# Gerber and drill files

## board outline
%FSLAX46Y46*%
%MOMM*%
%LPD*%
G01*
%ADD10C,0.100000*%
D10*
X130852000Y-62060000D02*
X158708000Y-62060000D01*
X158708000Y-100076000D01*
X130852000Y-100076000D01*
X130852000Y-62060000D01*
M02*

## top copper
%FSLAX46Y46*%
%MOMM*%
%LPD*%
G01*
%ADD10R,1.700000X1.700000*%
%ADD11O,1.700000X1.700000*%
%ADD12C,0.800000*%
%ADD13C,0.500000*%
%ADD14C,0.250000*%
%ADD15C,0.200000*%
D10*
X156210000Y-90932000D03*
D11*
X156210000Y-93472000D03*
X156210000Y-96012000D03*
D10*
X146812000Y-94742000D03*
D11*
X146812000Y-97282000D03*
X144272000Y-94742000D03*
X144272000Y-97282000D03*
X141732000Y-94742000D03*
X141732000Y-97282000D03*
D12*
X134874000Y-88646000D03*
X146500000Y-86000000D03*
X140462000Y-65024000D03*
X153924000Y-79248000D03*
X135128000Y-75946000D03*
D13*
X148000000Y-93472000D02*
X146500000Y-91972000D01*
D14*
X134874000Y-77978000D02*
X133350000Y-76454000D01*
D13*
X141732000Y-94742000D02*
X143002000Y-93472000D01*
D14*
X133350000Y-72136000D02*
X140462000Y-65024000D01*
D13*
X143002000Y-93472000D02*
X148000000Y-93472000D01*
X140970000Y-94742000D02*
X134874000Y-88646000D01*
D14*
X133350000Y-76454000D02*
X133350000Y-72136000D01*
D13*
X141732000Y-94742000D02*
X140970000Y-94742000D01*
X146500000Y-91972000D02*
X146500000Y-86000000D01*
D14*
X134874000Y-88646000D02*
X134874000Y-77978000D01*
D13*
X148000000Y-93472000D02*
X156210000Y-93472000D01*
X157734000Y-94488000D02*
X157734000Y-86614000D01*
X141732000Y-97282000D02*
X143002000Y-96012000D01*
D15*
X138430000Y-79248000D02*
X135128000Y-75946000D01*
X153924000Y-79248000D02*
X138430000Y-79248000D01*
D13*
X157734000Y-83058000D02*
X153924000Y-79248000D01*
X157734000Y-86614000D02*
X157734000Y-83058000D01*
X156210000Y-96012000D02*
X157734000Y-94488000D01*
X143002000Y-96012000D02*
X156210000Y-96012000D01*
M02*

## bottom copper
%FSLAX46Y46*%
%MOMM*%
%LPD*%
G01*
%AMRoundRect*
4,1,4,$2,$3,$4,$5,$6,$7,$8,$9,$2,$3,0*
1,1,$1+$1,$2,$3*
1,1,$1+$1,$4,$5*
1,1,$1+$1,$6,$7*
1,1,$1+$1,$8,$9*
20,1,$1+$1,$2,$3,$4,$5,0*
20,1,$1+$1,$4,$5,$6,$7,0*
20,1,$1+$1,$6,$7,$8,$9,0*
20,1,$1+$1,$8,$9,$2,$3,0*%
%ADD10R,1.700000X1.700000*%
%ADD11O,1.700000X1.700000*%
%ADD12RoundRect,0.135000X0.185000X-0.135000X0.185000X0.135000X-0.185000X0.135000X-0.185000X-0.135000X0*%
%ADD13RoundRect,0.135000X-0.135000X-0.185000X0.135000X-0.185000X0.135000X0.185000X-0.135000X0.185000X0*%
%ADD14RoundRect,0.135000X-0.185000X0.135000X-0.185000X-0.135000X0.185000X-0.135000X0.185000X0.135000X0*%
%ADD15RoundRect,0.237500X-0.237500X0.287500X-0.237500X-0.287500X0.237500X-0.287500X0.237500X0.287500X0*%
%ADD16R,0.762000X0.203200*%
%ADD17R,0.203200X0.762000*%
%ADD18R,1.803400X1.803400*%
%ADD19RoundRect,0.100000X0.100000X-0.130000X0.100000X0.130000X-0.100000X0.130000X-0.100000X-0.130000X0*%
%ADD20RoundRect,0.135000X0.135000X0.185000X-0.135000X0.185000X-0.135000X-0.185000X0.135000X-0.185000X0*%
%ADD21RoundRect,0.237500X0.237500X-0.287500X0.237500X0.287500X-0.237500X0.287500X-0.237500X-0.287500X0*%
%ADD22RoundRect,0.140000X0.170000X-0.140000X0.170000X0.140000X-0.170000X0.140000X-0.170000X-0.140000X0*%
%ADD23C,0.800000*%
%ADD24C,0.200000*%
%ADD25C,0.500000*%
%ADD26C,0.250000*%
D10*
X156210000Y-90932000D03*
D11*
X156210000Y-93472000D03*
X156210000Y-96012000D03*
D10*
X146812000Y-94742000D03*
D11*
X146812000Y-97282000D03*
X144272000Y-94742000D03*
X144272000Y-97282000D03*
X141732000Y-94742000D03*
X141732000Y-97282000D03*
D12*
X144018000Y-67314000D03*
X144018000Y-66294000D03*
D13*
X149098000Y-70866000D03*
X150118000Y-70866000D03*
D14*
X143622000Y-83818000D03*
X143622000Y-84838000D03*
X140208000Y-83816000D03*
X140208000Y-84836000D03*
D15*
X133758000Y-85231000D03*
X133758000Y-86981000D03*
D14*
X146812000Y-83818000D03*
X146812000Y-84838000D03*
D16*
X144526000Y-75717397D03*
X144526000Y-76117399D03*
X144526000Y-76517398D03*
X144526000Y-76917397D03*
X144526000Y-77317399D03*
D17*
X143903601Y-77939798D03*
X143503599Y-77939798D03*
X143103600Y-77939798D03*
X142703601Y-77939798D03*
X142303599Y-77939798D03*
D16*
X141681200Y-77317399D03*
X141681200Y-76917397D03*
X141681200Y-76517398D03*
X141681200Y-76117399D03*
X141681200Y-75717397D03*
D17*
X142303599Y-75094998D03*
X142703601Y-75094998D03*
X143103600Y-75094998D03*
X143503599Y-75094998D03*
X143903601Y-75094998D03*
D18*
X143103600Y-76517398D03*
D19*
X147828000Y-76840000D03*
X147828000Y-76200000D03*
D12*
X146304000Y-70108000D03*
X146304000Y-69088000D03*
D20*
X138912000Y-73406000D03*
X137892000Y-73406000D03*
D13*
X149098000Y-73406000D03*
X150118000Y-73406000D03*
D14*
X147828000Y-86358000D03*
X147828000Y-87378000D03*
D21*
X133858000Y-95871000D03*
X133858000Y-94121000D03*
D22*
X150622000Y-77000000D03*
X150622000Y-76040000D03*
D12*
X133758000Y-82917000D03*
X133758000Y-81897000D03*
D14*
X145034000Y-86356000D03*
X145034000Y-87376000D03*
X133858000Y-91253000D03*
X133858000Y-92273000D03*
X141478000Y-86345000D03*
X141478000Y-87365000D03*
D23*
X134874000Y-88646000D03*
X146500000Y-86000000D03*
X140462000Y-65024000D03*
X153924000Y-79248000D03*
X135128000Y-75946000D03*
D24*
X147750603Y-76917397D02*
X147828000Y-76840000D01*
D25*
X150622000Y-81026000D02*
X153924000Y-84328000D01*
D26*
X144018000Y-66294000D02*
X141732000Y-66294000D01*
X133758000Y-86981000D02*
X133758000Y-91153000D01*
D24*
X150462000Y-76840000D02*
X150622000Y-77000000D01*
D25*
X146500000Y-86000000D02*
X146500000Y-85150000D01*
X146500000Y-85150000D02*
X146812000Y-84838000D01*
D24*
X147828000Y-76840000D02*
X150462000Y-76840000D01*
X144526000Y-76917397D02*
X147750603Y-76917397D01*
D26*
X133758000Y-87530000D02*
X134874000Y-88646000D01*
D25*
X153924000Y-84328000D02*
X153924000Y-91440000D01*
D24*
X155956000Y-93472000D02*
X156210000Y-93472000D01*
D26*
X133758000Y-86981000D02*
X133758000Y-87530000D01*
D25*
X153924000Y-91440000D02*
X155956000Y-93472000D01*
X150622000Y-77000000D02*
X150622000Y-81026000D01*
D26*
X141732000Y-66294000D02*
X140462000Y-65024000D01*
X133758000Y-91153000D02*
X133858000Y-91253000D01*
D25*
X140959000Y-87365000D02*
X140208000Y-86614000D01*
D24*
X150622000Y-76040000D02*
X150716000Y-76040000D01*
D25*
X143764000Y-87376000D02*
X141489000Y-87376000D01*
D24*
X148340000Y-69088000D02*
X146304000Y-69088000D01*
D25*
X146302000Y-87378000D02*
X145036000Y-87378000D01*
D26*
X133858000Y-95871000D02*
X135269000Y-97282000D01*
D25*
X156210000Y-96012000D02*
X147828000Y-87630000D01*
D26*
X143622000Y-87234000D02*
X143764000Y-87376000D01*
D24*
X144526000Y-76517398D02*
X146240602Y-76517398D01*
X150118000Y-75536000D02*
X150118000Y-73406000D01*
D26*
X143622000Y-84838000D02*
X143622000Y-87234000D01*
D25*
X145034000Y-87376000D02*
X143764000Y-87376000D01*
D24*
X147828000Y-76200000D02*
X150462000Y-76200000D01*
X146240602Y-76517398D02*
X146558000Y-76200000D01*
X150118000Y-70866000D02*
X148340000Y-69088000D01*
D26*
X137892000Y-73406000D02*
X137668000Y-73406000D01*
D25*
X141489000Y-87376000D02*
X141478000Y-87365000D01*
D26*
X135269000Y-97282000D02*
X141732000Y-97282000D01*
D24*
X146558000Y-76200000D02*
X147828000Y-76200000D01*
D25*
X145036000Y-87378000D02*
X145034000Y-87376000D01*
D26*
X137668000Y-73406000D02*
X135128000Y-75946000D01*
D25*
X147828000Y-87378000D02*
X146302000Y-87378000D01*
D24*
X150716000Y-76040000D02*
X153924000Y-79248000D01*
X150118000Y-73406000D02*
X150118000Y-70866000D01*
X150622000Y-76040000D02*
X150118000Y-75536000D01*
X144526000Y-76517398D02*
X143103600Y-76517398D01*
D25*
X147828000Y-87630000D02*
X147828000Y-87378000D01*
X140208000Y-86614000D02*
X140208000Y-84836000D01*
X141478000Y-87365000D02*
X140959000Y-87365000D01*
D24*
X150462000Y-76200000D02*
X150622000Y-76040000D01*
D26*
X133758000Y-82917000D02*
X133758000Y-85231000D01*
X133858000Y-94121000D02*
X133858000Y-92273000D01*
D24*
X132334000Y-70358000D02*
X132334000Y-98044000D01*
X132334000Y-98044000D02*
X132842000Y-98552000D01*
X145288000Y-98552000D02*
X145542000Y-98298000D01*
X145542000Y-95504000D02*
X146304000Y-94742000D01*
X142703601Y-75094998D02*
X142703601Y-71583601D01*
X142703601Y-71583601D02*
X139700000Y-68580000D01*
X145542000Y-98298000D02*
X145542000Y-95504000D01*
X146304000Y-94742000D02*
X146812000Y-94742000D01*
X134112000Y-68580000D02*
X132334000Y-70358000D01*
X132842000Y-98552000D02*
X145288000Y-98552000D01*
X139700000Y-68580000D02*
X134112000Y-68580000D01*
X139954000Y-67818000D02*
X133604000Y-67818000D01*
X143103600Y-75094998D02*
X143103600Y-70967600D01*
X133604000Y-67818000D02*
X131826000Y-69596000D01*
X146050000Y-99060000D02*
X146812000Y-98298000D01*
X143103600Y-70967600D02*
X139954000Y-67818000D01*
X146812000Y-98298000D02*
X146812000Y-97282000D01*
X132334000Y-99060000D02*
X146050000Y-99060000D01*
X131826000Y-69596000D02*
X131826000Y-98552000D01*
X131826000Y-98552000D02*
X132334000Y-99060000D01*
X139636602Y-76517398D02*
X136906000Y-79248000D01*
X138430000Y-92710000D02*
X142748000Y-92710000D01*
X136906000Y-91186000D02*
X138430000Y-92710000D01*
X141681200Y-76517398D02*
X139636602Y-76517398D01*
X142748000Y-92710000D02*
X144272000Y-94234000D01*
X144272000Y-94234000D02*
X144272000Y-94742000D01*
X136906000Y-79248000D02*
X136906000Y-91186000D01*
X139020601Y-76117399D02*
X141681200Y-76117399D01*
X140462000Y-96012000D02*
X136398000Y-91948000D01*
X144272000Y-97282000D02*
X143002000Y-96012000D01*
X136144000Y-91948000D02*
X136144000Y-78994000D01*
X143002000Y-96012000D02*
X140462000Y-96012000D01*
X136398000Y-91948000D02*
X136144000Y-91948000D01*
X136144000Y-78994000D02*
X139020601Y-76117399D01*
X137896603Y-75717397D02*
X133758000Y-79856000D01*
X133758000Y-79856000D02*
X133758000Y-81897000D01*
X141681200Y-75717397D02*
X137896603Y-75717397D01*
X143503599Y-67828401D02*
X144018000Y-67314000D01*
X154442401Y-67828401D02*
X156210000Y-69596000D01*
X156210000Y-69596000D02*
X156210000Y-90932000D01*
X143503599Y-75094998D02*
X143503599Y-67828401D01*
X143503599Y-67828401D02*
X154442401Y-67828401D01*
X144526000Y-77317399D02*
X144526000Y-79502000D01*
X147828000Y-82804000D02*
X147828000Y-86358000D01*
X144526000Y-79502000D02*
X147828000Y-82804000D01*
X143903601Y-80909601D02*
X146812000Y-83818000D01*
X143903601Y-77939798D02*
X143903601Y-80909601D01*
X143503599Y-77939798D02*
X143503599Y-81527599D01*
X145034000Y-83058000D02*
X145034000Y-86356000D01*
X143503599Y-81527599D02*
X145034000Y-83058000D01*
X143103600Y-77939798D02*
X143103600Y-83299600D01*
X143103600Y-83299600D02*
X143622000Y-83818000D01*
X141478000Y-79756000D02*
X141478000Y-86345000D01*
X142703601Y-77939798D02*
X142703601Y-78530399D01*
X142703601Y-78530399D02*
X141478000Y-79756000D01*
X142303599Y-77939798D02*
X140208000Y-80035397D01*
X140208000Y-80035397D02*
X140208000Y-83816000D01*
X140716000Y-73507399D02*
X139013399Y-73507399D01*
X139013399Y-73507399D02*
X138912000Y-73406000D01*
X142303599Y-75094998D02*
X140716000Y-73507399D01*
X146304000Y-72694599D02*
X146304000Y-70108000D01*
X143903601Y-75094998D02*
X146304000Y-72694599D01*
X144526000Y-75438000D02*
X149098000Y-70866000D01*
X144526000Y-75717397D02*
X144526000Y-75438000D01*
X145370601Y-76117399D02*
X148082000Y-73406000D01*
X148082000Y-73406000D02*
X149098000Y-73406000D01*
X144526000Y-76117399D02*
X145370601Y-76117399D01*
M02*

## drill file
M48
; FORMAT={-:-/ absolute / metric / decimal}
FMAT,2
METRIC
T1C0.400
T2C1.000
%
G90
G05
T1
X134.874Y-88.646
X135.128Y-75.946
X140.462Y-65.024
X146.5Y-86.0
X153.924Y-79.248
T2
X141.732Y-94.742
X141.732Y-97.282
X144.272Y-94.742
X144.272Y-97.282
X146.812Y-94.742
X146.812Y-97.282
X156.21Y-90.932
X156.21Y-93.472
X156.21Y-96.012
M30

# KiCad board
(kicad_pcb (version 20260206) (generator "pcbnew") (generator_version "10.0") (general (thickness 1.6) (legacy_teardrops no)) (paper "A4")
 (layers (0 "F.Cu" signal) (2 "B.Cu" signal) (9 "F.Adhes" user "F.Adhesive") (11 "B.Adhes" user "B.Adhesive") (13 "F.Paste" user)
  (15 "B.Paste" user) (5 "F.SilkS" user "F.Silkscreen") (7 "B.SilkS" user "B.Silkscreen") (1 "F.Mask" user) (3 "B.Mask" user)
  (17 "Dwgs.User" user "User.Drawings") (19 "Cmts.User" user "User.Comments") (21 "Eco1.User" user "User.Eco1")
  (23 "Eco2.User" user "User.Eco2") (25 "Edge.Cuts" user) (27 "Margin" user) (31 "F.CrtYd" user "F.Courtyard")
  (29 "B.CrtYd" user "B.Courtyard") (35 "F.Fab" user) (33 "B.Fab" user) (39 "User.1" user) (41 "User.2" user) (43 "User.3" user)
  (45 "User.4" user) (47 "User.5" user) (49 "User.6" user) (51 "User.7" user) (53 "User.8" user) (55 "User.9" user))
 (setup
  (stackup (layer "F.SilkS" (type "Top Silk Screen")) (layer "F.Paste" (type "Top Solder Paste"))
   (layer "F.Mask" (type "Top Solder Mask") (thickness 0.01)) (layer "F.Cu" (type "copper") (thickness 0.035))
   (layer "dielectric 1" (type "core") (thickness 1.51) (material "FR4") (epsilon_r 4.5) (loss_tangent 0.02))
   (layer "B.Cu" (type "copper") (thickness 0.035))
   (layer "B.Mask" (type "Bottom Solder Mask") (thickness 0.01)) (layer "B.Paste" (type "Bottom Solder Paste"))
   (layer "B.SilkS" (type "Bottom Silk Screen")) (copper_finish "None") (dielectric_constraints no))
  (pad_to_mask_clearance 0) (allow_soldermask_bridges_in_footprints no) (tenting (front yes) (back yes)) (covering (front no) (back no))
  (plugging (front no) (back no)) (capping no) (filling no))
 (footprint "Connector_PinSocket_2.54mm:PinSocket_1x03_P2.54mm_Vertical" (layer "F.Cu") (at 156.21 90.932)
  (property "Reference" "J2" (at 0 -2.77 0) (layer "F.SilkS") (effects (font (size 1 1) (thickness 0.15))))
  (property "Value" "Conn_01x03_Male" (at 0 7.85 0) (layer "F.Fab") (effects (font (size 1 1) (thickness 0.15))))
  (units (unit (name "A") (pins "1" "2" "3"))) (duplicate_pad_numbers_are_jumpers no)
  (pad "1" thru_hole rect (at 0 0) (size 1.7 1.7) (drill 1) (layers "*.Cu" "*.Mask") (remove_unused_layers no) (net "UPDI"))
  (pad "2" thru_hole oval (at 0 2.54) (size 1.7 1.7) (drill 1) (layers "*.Cu" "*.Mask") (remove_unused_layers no) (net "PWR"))
  (pad "3" thru_hole oval (at 0 5.08) (size 1.7 1.7) (drill 1) (layers "*.Cu" "*.Mask") (remove_unused_layers no) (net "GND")))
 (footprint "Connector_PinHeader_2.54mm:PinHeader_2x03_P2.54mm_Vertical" (layer "F.Cu") (at 146.812 94.742 -90)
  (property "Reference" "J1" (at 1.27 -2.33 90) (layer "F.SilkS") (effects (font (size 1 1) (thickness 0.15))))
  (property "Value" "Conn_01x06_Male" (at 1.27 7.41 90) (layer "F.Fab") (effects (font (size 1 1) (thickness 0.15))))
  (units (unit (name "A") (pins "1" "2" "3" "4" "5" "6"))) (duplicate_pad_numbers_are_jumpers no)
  (pad "1" thru_hole rect (at 0 0 270) (size 1.7 1.7) (drill 1) (layers "*.Cu" "*.Mask") (remove_unused_layers no) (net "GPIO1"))
  (pad "2" thru_hole oval (at 2.54 0 270) (size 1.7 1.7) (drill 1) (layers "*.Cu" "*.Mask") (remove_unused_layers no) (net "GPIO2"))
  (pad "3" thru_hole oval (at 0 2.54 270) (size 1.7 1.7) (drill 1) (layers "*.Cu" "*.Mask") (remove_unused_layers no) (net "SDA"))
  (pad "4" thru_hole oval (at 2.54 2.54 270) (size 1.7 1.7) (drill 1) (layers "*.Cu" "*.Mask") (remove_unused_layers no) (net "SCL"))
  (pad "5" thru_hole oval (at 0 5.08 270) (size 1.7 1.7) (drill 1) (layers "*.Cu" "*.Mask") (remove_unused_layers no) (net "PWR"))
  (pad "6" thru_hole oval (at 2.54 5.08 270) (size 1.7 1.7) (drill 1) (layers "*.Cu" "*.Mask") (remove_unused_layers no) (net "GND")))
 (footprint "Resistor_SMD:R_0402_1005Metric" (layer "B.Cu") (at 144.018 66.804 90)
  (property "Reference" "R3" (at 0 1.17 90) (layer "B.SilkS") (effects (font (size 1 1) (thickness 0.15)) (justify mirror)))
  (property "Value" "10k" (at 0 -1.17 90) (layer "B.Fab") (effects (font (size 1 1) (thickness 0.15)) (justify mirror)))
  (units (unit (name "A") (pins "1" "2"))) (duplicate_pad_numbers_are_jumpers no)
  (pad "1" smd roundrect (at -0.51 0 90) (size 0.54 0.64) (layers "B.Cu" "B.Mask" "B.Paste") (roundrect_rratio 0.25) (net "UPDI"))
  (pad "2" smd roundrect (at 0.51 0 90) (size 0.54 0.64) (layers "B.Cu" "B.Mask" "B.Paste") (roundrect_rratio 0.25) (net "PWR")))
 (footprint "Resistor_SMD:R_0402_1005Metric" (layer "B.Cu") (at 149.608 70.866)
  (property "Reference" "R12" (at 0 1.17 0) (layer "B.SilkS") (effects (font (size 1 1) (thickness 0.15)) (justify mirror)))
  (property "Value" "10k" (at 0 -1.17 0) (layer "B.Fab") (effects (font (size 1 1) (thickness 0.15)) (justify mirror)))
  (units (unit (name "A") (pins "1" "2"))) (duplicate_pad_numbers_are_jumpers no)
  (pad "1" smd roundrect (at -0.51 0) (size 0.54 0.64) (layers "B.Cu" "B.Mask" "B.Paste") (roundrect_rratio 0.25) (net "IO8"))
  (pad "2" smd roundrect (at 0.51 0) (size 0.54 0.64) (layers "B.Cu" "B.Mask" "B.Paste") (roundrect_rratio 0.25) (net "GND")))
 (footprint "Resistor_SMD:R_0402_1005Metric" (layer "B.Cu") (at 143.622 84.328 -90)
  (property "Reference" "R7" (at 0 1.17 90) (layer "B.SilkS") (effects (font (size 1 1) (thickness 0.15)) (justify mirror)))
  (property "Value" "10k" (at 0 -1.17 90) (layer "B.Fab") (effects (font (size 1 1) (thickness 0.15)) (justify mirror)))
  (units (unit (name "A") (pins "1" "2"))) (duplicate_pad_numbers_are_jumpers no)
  (pad "1" smd roundrect (at -0.51 0 270) (size 0.54 0.64) (layers "B.Cu" "B.Mask" "B.Paste") (roundrect_rratio 0.25) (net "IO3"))
  (pad "2" smd roundrect (at 0.51 0 270) (size 0.54 0.64) (layers "B.Cu" "B.Mask" "B.Paste") (roundrect_rratio 0.25) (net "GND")))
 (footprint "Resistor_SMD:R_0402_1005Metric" (layer "B.Cu") (at 140.208 84.326 -90)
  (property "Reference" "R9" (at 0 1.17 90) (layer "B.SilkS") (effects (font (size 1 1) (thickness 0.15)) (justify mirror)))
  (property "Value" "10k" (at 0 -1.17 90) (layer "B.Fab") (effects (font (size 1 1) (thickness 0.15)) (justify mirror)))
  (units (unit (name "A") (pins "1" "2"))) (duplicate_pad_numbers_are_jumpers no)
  (pad "1" smd roundrect (at -0.51 0 270) (size 0.54 0.64) (layers "B.Cu" "B.Mask" "B.Paste") (roundrect_rratio 0.25) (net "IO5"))
  (pad "2" smd roundrect (at 0.51 0 270) (size 0.54 0.64) (layers "B.Cu" "B.Mask" "B.Paste") (roundrect_rratio 0.25) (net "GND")))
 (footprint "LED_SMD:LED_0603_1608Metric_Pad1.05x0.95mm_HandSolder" (layer "B.Cu") (at 133.758 86.106 -90)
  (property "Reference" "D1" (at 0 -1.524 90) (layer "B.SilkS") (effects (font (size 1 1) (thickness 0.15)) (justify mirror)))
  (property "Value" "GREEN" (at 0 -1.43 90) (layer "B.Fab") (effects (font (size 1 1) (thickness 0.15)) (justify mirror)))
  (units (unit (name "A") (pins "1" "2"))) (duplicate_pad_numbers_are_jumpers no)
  (pad "1" smd roundrect (at -0.875 0 270) (size 1.05 0.95) (layers "B.Cu" "B.Mask" "B.Paste") (roundrect_rratio 0.25) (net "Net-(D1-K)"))
  (pad "2" smd roundrect (at 0.875 0 270) (size 1.05 0.95) (layers "B.Cu" "B.Mask" "B.Paste") (roundrect_rratio 0.25) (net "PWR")))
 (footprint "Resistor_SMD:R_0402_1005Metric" (layer "B.Cu") (at 146.812 84.328 -90)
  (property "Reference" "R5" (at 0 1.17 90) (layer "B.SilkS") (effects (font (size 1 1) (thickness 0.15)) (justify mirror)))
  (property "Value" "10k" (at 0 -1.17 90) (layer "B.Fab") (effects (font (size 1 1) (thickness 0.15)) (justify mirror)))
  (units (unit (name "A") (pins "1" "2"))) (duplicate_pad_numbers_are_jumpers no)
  (pad "1" smd roundrect (at -0.51 0 270) (size 0.54 0.64) (layers "B.Cu" "B.Mask" "B.Paste") (roundrect_rratio 0.25) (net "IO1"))
  (pad "2" smd roundrect (at 0.51 0 270) (size 0.54 0.64) (layers "B.Cu" "B.Mask" "B.Paste") (roundrect_rratio 0.25) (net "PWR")))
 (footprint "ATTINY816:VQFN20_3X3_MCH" (layer "B.Cu") (at 143.1036 76.517398 180)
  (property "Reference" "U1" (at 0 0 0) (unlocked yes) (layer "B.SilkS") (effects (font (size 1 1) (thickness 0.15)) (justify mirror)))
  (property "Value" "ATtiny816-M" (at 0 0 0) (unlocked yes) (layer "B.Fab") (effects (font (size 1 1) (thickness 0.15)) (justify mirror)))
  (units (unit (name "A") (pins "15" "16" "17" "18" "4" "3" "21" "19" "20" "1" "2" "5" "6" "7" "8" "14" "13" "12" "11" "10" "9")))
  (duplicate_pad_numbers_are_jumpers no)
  (pad "1" smd rect (at -1.4224 0.800001 90) (size 0.2032 0.762) (layers "B.Cu" "B.Mask" "B.Paste") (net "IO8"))
  (pad "2" smd rect (at -1.4224 0.399999 90) (size 0.2032 0.762) (layers "B.Cu" "B.Mask" "B.Paste") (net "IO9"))
  (pad "3" smd rect (at -1.4224 0 90) (size 0.2032 0.762) (layers "B.Cu" "B.Mask" "B.Paste") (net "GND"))
  (pad "4" smd rect (at -1.4224 -0.399999 90) (size 0.2032 0.762) (layers "B.Cu" "B.Mask" "B.Paste") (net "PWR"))
  (pad "5" smd rect (at -1.4224 -0.800001 90) (size 0.2032 0.762) (layers "B.Cu" "B.Mask" "B.Paste") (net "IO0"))
  (pad "6" smd rect (at -0.800001 -1.4224 180) (size 0.2032 0.762) (layers "B.Cu" "B.Mask" "B.Paste") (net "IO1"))
  (pad "7" smd rect (at -0.399999 -1.4224 180) (size 0.2032 0.762) (layers "B.Cu" "B.Mask" "B.Paste") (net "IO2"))
  (pad "8" smd rect (at 0 -1.4224 180) (size 0.2032 0.762) (layers "B.Cu" "B.Mask" "B.Paste") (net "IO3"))
  (pad "9" smd rect (at 0.399999 -1.4224 180) (size 0.2032 0.762) (layers "B.Cu" "B.Mask" "B.Paste") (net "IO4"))
  (pad "10" smd rect (at 0.800001 -1.4224 180) (size 0.2032 0.762) (layers "B.Cu" "B.Mask" "B.Paste") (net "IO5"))
  (pad "11" smd rect (at 1.4224 -0.800001 90) (size 0.2032 0.762) (layers "B.Cu" "B.Mask" "B.Paste") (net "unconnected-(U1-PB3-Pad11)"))
  (pad "12" smd rect (at 1.4224 -0.399999 90) (size 0.2032 0.762) (layers "B.Cu" "B.Mask" "B.Paste") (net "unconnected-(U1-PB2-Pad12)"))
  (pad "13" smd rect (at 1.4224 0 90) (size 0.2032 0.762) (layers "B.Cu" "B.Mask" "B.Paste") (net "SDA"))
  (pad "14" smd rect (at 1.4224 0.399999 90) (size 0.2032 0.762) (layers "B.Cu" "B.Mask" "B.Paste") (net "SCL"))
  (pad "15" smd rect (at 1.4224 0.800001 90) (size 0.2032 0.762) (layers "B.Cu" "B.Mask" "B.Paste") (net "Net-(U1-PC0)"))
  (pad "16" smd rect (at 0.800001 1.4224 180) (size 0.2032 0.762) (layers "B.Cu" "B.Mask" "B.Paste") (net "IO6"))
  (pad "17" smd rect (at 0.399999 1.4224 180) (size 0.2032 0.762) (layers "B.Cu" "B.Mask" "B.Paste") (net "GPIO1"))
  (pad "18" smd rect (at 0 1.4224 180) (size 0.2032 0.762) (layers "B.Cu" "B.Mask" "B.Paste") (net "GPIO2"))
  (pad "19" smd rect (at -0.399999 1.4224 180) (size 0.2032 0.762) (layers "B.Cu" "B.Mask" "B.Paste") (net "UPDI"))
  (pad "20" smd rect (at -0.800001 1.4224 180) (size 0.2032 0.762) (layers "B.Cu" "B.Mask" "B.Paste") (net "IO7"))
  (pad "21" smd rect (at 0 0 180) (size 1.8034 1.8034) (layers "B.Cu" "B.Mask" "B.Paste") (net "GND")))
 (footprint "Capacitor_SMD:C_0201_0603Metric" (layer "B.Cu") (at 147.828 76.52 90)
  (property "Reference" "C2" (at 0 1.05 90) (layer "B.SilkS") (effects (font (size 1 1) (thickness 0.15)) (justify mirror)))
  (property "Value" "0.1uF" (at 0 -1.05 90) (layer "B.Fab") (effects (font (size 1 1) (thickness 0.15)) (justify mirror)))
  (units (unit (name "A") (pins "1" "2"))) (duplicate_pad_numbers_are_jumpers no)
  (pad "" smd roundrect (at -0.345 0 90) (size 0.318 0.36) (layers "B.Paste") (roundrect_rratio 0.25))
  (pad "" smd roundrect (at 0.345 0 90) (size 0.318 0.36) (layers "B.Paste") (roundrect_rratio 0.25))
  (pad "1" smd roundrect (at -0.32 0 90) (size 0.46 0.4) (layers "B.Cu" "B.Mask") (roundrect_rratio 0.25) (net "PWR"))
  (pad "2" smd roundrect (at 0.32 0 90) (size 0.46 0.4) (layers "B.Cu" "B.Mask") (roundrect_rratio 0.25) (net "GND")))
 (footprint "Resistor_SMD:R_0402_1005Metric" (layer "B.Cu") (at 146.304 69.598 90)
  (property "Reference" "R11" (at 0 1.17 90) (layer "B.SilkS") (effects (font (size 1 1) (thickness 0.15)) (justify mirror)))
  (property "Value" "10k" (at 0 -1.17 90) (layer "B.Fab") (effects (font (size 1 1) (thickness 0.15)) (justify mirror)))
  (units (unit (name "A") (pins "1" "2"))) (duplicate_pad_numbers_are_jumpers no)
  (pad "1" smd roundrect (at -0.51 0 90) (size 0.54 0.64) (layers "B.Cu" "B.Mask" "B.Paste") (roundrect_rratio 0.25) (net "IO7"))
  (pad "2" smd roundrect (at 0.51 0 90) (size 0.54 0.64) (layers "B.Cu" "B.Mask" "B.Paste") (roundrect_rratio 0.25) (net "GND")))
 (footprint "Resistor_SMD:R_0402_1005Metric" (layer "B.Cu") (at 138.402 73.406 180)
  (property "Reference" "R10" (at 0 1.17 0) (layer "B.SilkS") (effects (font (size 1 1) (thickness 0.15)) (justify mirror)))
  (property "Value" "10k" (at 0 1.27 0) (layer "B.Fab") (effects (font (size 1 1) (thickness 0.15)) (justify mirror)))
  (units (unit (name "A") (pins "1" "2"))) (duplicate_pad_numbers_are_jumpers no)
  (pad "1" smd roundrect (at -0.51 0 180) (size 0.54 0.64) (layers "B.Cu" "B.Mask" "B.Paste") (roundrect_rratio 0.25) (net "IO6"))
  (pad "2" smd roundrect (at 0.51 0 180) (size 0.54 0.64) (layers "B.Cu" "B.Mask" "B.Paste") (roundrect_rratio 0.25) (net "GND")))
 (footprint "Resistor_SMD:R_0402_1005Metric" (layer "B.Cu") (at 149.608 73.406)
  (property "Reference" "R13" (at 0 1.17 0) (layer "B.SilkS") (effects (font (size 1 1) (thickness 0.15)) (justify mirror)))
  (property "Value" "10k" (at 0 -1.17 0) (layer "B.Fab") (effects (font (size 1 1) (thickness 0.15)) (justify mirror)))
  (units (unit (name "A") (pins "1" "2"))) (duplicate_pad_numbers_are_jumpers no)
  (pad "1" smd roundrect (at -0.51 0) (size 0.54 0.64) (layers "B.Cu" "B.Mask" "B.Paste") (roundrect_rratio 0.25) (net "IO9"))
  (pad "2" smd roundrect (at 0.51 0) (size 0.54 0.64) (layers "B.Cu" "B.Mask" "B.Paste") (roundrect_rratio 0.25) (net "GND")))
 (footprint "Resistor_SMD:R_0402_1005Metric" (layer "B.Cu") (at 147.828 86.868 -90)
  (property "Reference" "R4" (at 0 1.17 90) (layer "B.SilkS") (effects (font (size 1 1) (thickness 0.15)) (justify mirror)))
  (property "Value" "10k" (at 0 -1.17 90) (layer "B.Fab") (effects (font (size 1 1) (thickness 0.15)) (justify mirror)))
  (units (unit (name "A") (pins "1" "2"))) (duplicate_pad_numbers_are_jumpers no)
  (pad "1" smd roundrect (at -0.51 0 270) (size 0.54 0.64) (layers "B.Cu" "B.Mask" "B.Paste") (roundrect_rratio 0.25) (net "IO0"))
  (pad "2" smd roundrect (at 0.51 0 270) (size 0.54 0.64) (layers "B.Cu" "B.Mask" "B.Paste") (roundrect_rratio 0.25) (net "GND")))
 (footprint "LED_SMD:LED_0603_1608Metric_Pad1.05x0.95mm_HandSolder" (layer "B.Cu") (at 133.858 94.996 90)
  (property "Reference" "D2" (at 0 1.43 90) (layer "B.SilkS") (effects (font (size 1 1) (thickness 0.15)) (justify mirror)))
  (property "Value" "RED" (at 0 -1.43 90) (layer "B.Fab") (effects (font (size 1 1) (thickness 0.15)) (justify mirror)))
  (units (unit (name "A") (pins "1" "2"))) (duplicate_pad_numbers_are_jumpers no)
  (pad "1" smd roundrect (at -0.875 0 90) (size 1.05 0.95) (layers "B.Cu" "B.Mask" "B.Paste") (roundrect_rratio 0.25) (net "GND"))
  (pad "2" smd roundrect (at 0.875 0 90) (size 1.05 0.95) (layers "B.Cu" "B.Mask" "B.Paste") (roundrect_rratio 0.25) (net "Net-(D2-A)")))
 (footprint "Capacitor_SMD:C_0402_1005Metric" (layer "B.Cu") (at 150.622 76.52 90)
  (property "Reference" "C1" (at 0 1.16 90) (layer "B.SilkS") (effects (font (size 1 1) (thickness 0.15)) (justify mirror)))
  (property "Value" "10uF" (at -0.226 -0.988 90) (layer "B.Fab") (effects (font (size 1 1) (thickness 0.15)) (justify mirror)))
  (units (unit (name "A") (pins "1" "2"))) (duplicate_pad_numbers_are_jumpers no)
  (pad "1" smd roundrect (at -0.48 0 90) (size 0.56 0.62) (layers "B.Cu" "B.Mask" "B.Paste") (roundrect_rratio 0.25) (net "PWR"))
  (pad "2" smd roundrect (at 0.48 0 90) (size 0.56 0.62) (layers "B.Cu" "B.Mask" "B.Paste") (roundrect_rratio 0.25) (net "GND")))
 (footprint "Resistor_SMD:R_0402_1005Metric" (layer "B.Cu") (at 133.758 82.407 90)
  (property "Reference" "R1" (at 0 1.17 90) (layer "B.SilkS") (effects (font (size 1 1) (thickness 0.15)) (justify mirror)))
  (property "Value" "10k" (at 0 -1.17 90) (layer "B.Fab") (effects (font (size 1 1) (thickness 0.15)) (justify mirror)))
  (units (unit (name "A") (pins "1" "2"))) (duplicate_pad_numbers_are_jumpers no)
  (pad "1" smd roundrect (at -0.51 0 90) (size 0.54 0.64) (layers "B.Cu" "B.Mask" "B.Paste") (roundrect_rratio 0.25) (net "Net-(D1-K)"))
  (pad "2" smd roundrect (at 0.51 0 90) (size 0.54 0.64) (layers "B.Cu" "B.Mask" "B.Paste") (roundrect_rratio 0.25) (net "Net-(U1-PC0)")))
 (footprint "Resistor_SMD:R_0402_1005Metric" (layer "B.Cu") (at 145.034 86.866 -90)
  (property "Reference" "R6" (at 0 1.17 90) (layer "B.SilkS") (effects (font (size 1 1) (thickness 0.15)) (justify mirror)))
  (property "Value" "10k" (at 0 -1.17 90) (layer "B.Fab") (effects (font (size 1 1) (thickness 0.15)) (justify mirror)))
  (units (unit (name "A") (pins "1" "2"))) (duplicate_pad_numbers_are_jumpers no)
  (pad "1" smd roundrect (at -0.51 0 270) (size 0.54 0.64) (layers "B.Cu" "B.Mask" "B.Paste") (roundrect_rratio 0.25) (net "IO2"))
  (pad "2" smd roundrect (at 0.51 0 270) (size 0.54 0.64) (layers "B.Cu" "B.Mask" "B.Paste") (roundrect_rratio 0.25) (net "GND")))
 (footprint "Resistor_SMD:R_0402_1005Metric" (layer "B.Cu") (at 133.858 91.763 -90)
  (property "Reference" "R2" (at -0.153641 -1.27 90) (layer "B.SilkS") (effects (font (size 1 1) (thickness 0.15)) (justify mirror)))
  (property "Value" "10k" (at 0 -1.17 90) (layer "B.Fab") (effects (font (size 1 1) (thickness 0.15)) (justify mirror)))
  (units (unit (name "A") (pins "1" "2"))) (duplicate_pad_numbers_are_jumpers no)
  (pad "1" smd roundrect (at -0.51 0 270) (size 0.54 0.64) (layers "B.Cu" "B.Mask" "B.Paste") (roundrect_rratio 0.25) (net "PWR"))
  (pad "2" smd roundrect (at 0.51 0 270) (size 0.54 0.64) (layers "B.Cu" "B.Mask" "B.Paste") (roundrect_rratio 0.25) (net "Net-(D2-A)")))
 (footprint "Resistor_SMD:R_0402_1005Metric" (layer "B.Cu") (at 141.478 86.855 -90)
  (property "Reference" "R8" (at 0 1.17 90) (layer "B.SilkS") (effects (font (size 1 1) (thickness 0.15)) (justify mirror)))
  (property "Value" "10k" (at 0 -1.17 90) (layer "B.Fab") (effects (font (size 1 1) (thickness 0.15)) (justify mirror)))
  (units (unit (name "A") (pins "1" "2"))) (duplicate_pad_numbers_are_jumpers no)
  (pad "1" smd roundrect (at -0.51 0 270) (size 0.54 0.64) (layers "B.Cu" "B.Mask" "B.Paste") (roundrect_rratio 0.25) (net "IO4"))
  (pad "2" smd roundrect (at 0.51 0 270) (size 0.54 0.64) (layers "B.Cu" "B.Mask" "B.Paste") (roundrect_rratio 0.25) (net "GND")))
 (gr_rect (start 130.852 62.06) (end 158.708 100.076) (stroke (width 0.1) (type solid)) (fill no) (layer "Edge.Cuts"))
 (via (at 134.874 88.646) (size 0.8) (drill 0.4) (layers "F.Cu" "B.Cu") (free yes) (capping no) (covering (front no) (back no))
  (plugging (front no) (back no)) (filling no) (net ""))
 (segment (start 148 93.472) (end 146.5 91.972) (width 0.5) (layer "F.Cu") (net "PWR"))
 (segment (start 134.874 77.978) (end 133.35 76.454) (width 0.25) (layer "F.Cu") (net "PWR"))
 (segment (start 141.732 94.742) (end 143.002 93.472) (width 0.5) (layer "F.Cu") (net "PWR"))
 (segment (start 133.35 72.136) (end 140.462 65.024) (width 0.25) (layer "F.Cu") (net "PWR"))
 (segment (start 143.002 93.472) (end 148 93.472) (width 0.5) (layer "F.Cu") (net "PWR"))
 (segment (start 140.97 94.742) (end 134.874 88.646) (width 0.5) (layer "F.Cu") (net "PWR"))
 (segment (start 133.35 76.454) (end 133.35 72.136) (width 0.25) (layer "F.Cu") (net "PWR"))
 (segment (start 141.732 94.742) (end 140.97 94.742) (width 0.5) (layer "F.Cu") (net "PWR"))
 (segment (start 146.5 91.972) (end 146.5 86) (width 0.5) (layer "F.Cu") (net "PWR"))
 (segment (start 134.874 88.646) (end 134.874 77.978) (width 0.25) (layer "F.Cu") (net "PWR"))
 (segment (start 148 93.472) (end 156.21 93.472) (width 0.5) (layer "F.Cu") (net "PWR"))
 (via (at 146.5 86) (size 0.8) (drill 0.4) (layers "F.Cu" "B.Cu") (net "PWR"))
 (via (at 140.462 65.024) (size 0.8) (drill 0.4) (layers "F.Cu" "B.Cu") (capping no) (covering (front no) (back no))
  (plugging (front no) (back no)) (filling no) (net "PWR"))
 (segment (start 147.750603 76.917397) (end 147.828 76.84) (width 0.2) (layer "B.Cu") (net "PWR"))
 (segment (start 150.622 81.026) (end 153.924 84.328) (width 0.5) (layer "B.Cu") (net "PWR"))
 (segment (start 144.018 66.294) (end 141.732 66.294) (width 0.25) (layer "B.Cu") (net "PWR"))
 (segment (start 133.758 86.981) (end 133.758 91.153) (width 0.25) (layer "B.Cu") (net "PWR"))
 (segment (start 150.462 76.84) (end 150.622 77) (width 0.2) (layer "B.Cu") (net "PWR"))
 (segment (start 146.5 86) (end 146.5 85.15) (width 0.5) (layer "B.Cu") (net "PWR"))
 (segment (start 146.5 85.15) (end 146.812 84.838) (width 0.5) (layer "B.Cu") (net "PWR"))
 (segment (start 147.828 76.84) (end 150.462 76.84) (width 0.2) (layer "B.Cu") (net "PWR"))
 (segment (start 144.526 76.917397) (end 147.750603 76.917397) (width 0.2) (layer "B.Cu") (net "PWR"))
 (segment (start 133.758 87.53) (end 134.874 88.646) (width 0.25) (layer "B.Cu") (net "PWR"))
 (segment (start 153.924 84.328) (end 153.924 91.44) (width 0.5) (layer "B.Cu") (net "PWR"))
 (segment (start 155.956 93.472) (end 156.21 93.472) (width 0.2) (layer "B.Cu") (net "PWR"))
 (segment (start 133.758 86.981) (end 133.758 87.53) (width 0.25) (layer "B.Cu") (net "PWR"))
 (segment (start 153.924 91.44) (end 155.956 93.472) (width 0.5) (layer "B.Cu") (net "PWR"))
 (segment (start 150.622 77) (end 150.622 81.026) (width 0.5) (layer "B.Cu") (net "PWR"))
 (segment (start 141.732 66.294) (end 140.462 65.024) (width 0.25) (layer "B.Cu") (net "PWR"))
 (segment (start 133.758 91.153) (end 133.858 91.253) (width 0.25) (layer "B.Cu") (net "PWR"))
 (segment (start 157.734 94.488) (end 157.734 86.614) (width 0.5) (layer "F.Cu") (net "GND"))
 (segment (start 141.732 97.282) (end 143.002 96.012) (width 0.5) (layer "F.Cu") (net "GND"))
 (segment (start 138.43 79.248) (end 135.128 75.946) (width 0.2) (layer "F.Cu") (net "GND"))
 (segment (start 153.924 79.248) (end 138.43 79.248) (width 0.2) (layer "F.Cu") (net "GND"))
 (segment (start 157.734 83.058) (end 153.924 79.248) (width 0.5) (layer "F.Cu") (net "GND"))
 (segment (start 157.734 86.614) (end 157.734 83.058) (width 0.5) (layer "F.Cu") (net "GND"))
 (segment (start 156.21 96.012) (end 157.734 94.488) (width 0.5) (layer "F.Cu") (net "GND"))
 (segment (start 143.002 96.012) (end 156.21 96.012) (width 0.5) (layer "F.Cu") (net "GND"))
 (via (at 153.924 79.248) (size 0.8) (drill 0.4) (layers "F.Cu" "B.Cu") (capping no) (covering (front no) (back no))
  (plugging (front no) (back no)) (filling no) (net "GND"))
 (via (at 135.128 75.946) (size 0.8) (drill 0.4) (layers "F.Cu" "B.Cu") (capping no) (covering (front no) (back no))
  (plugging (front no) (back no)) (filling no) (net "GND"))
 (segment (start 140.959 87.365) (end 140.208 86.614) (width 0.5) (layer "B.Cu") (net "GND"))
 (segment (start 150.622 76.04) (end 150.716 76.04) (width 0.2) (layer "B.Cu") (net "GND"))
 (segment (start 143.764 87.376) (end 141.489 87.376) (width 0.5) (layer "B.Cu") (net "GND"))
 (segment (start 148.34 69.088) (end 146.304 69.088) (width 0.2) (layer "B.Cu") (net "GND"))
 (segment (start 146.302 87.378) (end 145.036 87.378) (width 0.5) (layer "B.Cu") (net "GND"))
 (segment (start 133.858 95.871) (end 135.269 97.282) (width 0.25) (layer "B.Cu") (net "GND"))
 (segment (start 156.21 96.012) (end 147.828 87.63) (width 0.5) (layer "B.Cu") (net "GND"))
 (segment (start 143.622 87.234) (end 143.764 87.376) (width 0.25) (layer "B.Cu") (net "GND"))
 (segment (start 144.526 76.517398) (end 146.240602 76.517398) (width 0.2) (layer "B.Cu") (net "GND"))
 (segment (start 150.118 75.536) (end 150.118 73.406) (width 0.2) (layer "B.Cu") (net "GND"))
 (segment (start 143.622 84.838) (end 143.622 87.234) (width 0.25) (layer "B.Cu") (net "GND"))
 (segment (start 145.034 87.376) (end 143.764 87.376) (width 0.5) (layer "B.Cu") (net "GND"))
 (segment (start 147.828 76.2) (end 150.462 76.2) (width 0.2) (layer "B.Cu") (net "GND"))
 (segment (start 146.240602 76.517398) (end 146.558 76.2) (width 0.2) (layer "B.Cu") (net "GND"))
 (segment (start 150.118 70.866) (end 148.34 69.088) (width 0.2) (layer "B.Cu") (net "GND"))
 (segment (start 137.892 73.406) (end 137.668 73.406) (width 0.25) (layer "B.Cu") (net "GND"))
 (segment (start 141.489 87.376) (end 141.478 87.365) (width 0.5) (layer "B.Cu") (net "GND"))
 (segment (start 135.269 97.282) (end 141.732 97.282) (width 0.25) (layer "B.Cu") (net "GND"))
 (segment (start 146.558 76.2) (end 147.828 76.2) (width 0.2) (layer "B.Cu") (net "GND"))
 (segment (start 145.036 87.378) (end 145.034 87.376) (width 0.5) (layer "B.Cu") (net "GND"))
 (segment (start 137.668 73.406) (end 135.128 75.946) (width 0.25) (layer "B.Cu") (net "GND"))
 (segment (start 147.828 87.378) (end 146.302 87.378) (width 0.5) (layer "B.Cu") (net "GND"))
 (segment (start 150.716 76.04) (end 153.924 79.248) (width 0.2) (layer "B.Cu") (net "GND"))
 (segment (start 150.118 73.406) (end 150.118 70.866) (width 0.2) (layer "B.Cu") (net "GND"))
 (segment (start 150.622 76.04) (end 150.118 75.536) (width 0.2) (layer "B.Cu") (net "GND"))
 (segment (start 144.526 76.517398) (end 143.1036 76.517398) (width 0.2) (layer "B.Cu") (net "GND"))
 (segment (start 147.828 87.63) (end 147.828 87.378) (width 0.5) (layer "B.Cu") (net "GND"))
 (segment (start 140.208 86.614) (end 140.208 84.836) (width 0.5) (layer "B.Cu") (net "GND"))
 (segment (start 141.478 87.365) (end 140.959 87.365) (width 0.5) (layer "B.Cu") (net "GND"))
 (segment (start 150.462 76.2) (end 150.622 76.04) (width 0.2) (layer "B.Cu") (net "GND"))
 (segment (start 133.758 82.917) (end 133.758 85.231) (width 0.25) (layer "B.Cu") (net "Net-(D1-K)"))
 (segment (start 133.858 94.121) (end 133.858 92.273) (width 0.25) (layer "B.Cu") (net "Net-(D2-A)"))
 (segment (start 132.334 70.358) (end 132.334 98.044) (width 0.2) (layer "B.Cu") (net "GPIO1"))
 (segment (start 132.334 98.044) (end 132.842 98.552) (width 0.2) (layer "B.Cu") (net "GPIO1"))
 (segment (start 145.288 98.552) (end 145.542 98.298) (width 0.2) (layer "B.Cu") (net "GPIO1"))
 (segment (start 145.542 95.504) (end 146.304 94.742) (width 0.2) (layer "B.Cu") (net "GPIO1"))
 (segment (start 142.703601 75.094998) (end 142.703601 71.583601) (width 0.2) (layer "B.Cu") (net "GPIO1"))
 (segment (start 142.703601 71.583601) (end 139.7 68.58) (width 0.2) (layer "B.Cu") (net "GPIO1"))
 (segment (start 145.542 98.298) (end 145.542 95.504) (width 0.2) (layer "B.Cu") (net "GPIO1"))
 (segment (start 146.304 94.742) (end 146.812 94.742) (width 0.2) (layer "B.Cu") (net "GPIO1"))
 (segment (start 134.112 68.58) (end 132.334 70.358) (width 0.2) (layer "B.Cu") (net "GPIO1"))
 (segment (start 132.842 98.552) (end 145.288 98.552) (width 0.2) (layer "B.Cu") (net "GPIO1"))
 (segment (start 139.7 68.58) (end 134.112 68.58) (width 0.2) (layer "B.Cu") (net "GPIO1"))
 (segment (start 139.954 67.818) (end 133.604 67.818) (width 0.2) (layer "B.Cu") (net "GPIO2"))
 (segment (start 143.1036 75.094998) (end 143.1036 70.9676) (width 0.2) (layer "B.Cu") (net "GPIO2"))
 (segment (start 133.604 67.818) (end 131.826 69.596) (width 0.2) (layer "B.Cu") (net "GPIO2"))
 (segment (start 146.05 99.06) (end 146.812 98.298) (width 0.2) (layer "B.Cu") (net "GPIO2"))
 (segment (start 143.1036 70.9676) (end 139.954 67.818) (width 0.2) (layer "B.Cu") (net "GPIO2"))
 (segment (start 146.812 98.298) (end 146.812 97.282) (width 0.2) (layer "B.Cu") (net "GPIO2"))
 (segment (start 132.334 99.06) (end 146.05 99.06) (width 0.2) (layer "B.Cu") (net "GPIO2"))
 (segment (start 131.826 69.596) (end 131.826 98.552) (width 0.2) (layer "B.Cu") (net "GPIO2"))
 (segment (start 131.826 98.552) (end 132.334 99.06) (width 0.2) (layer "B.Cu") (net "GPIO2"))
 (segment (start 139.636602 76.517398) (end 136.906 79.248) (width 0.2) (layer "B.Cu") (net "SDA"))
 (segment (start 138.43 92.71) (end 142.748 92.71) (width 0.2) (layer "B.Cu") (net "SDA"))
 (segment (start 136.906 91.186) (end 138.43 92.71) (width 0.2) (layer "B.Cu") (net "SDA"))
 (segment (start 141.6812 76.517398) (end 139.636602 76.517398) (width 0.2) (layer "B.Cu") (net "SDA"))
 (segment (start 142.748 92.71) (end 144.272 94.234) (width 0.2) (layer "B.Cu") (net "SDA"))
 (segment (start 144.272 94.234) (end 144.272 94.742) (width 0.2) (layer "B.Cu") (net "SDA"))
 (segment (start 136.906 79.248) (end 136.906 91.186) (width 0.2) (layer "B.Cu") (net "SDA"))
 (segment (start 139.020601 76.117399) (end 141.6812 76.117399) (width 0.2) (layer "B.Cu") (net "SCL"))
 (segment (start 140.462 96.012) (end 136.398 91.948) (width 0.2) (layer "B.Cu") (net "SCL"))
 (segment (start 144.272 97.282) (end 143.002 96.012) (width 0.2) (layer "B.Cu") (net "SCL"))
 (segment (start 136.144 91.948) (end 136.144 78.994) (width 0.2) (layer "B.Cu") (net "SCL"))
 (segment (start 143.002 96.012) (end 140.462 96.012) (width 0.2) (layer "B.Cu") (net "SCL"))
 (segment (start 136.398 91.948) (end 136.144 91.948) (width 0.2) (layer "B.Cu") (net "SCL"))
 (segment (start 136.144 78.994) (end 139.020601 76.117399) (width 0.2) (layer "B.Cu") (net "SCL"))
 (segment (start 137.896603 75.717397) (end 133.758 79.856) (width 0.2) (layer "B.Cu") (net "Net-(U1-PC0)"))
 (segment (start 133.758 79.856) (end 133.758 81.897) (width 0.2) (layer "B.Cu") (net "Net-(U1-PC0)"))
 (segment (start 141.6812 75.717397) (end 137.896603 75.717397) (width 0.2) (layer "B.Cu") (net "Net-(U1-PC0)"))
 (segment (start 143.503599 67.828401) (end 144.018 67.314) (width 0.2) (layer "B.Cu") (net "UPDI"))
 (segment (start 154.442401 67.828401) (end 156.21 69.596) (width 0.2) (layer "B.Cu") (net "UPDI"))
 (segment (start 156.21 69.596) (end 156.21 90.932) (width 0.2) (layer "B.Cu") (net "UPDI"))
 (segment (start 143.503599 75.094998) (end 143.503599 67.828401) (width 0.2) (layer "B.Cu") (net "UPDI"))
 (segment (start 143.503599 67.828401) (end 154.442401 67.828401) (width 0.2) (layer "B.Cu") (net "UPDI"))
 (segment (start 144.526 77.317399) (end 144.526 79.502) (width 0.2) (layer "B.Cu") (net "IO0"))
 (segment (start 147.828 82.804) (end 147.828 86.358) (width 0.2) (layer "B.Cu") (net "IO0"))
 (segment (start 144.526 79.502) (end 147.828 82.804) (width 0.2) (layer "B.Cu") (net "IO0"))
 (segment (start 143.903601 80.909601) (end 146.812 83.818) (width 0.2) (layer "B.Cu") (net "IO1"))
 (segment (start 143.903601 77.939798) (end 143.903601 80.909601) (width 0.2) (layer "B.Cu") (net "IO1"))
 (segment (start 143.503599 77.939798) (end 143.503599 81.527599) (width 0.2) (layer "B.Cu") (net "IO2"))
 (segment (start 145.034 83.058) (end 145.034 86.356) (width 0.2) (layer "B.Cu") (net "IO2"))
 (segment (start 143.503599 81.527599) (end 145.034 83.058) (width 0.2) (layer "B.Cu") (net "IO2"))
 (segment (start 143.1036 77.939798) (end 143.1036 83.2996) (width 0.2) (layer "B.Cu") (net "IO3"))
 (segment (start 143.1036 83.2996) (end 143.622 83.818) (width 0.2) (layer "B.Cu") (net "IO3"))
 (segment (start 141.478 79.756) (end 141.478 86.345) (width 0.2) (layer "B.Cu") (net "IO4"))
 (segment (start 142.703601 77.939798) (end 142.703601 78.530399) (width 0.2) (layer "B.Cu") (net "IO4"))
 (segment (start 142.703601 78.530399) (end 141.478 79.756) (width 0.2) (layer "B.Cu") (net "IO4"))
 (segment (start 142.303599 77.939798) (end 140.208 80.035397) (width 0.2) (layer "B.Cu") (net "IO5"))
 (segment (start 140.208 80.035397) (end 140.208 83.816) (width 0.2) (layer "B.Cu") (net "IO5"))
 (segment (start 140.716 73.507399) (end 139.013399 73.507399) (width 0.2) (layer "B.Cu") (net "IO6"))
 (segment (start 139.013399 73.507399) (end 138.912 73.406) (width 0.2) (layer "B.Cu") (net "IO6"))
 (segment (start 142.303599 75.094998) (end 140.716 73.507399) (width 0.2) (layer "B.Cu") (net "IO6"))
 (segment (start 146.304 72.694599) (end 146.304 70.108) (width 0.2) (layer "B.Cu") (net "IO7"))
 (segment (start 143.903601 75.094998) (end 146.304 72.694599) (width 0.2) (layer "B.Cu") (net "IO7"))
 (segment (start 144.526 75.438) (end 149.098 70.866) (width 0.2) (layer "B.Cu") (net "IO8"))
 (segment (start 144.526 75.717397) (end 144.526 75.438) (width 0.2) (layer "B.Cu") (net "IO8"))
 (segment (start 145.370601 76.117399) (end 148.082 73.406) (width 0.2) (layer "B.Cu") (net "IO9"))
 (segment (start 148.082 73.406) (end 149.098 73.406) (width 0.2) (layer "B.Cu") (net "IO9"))
 (segment (start 144.526 76.117399) (end 145.370601 76.117399) (width 0.2) (layer "B.Cu") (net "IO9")))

